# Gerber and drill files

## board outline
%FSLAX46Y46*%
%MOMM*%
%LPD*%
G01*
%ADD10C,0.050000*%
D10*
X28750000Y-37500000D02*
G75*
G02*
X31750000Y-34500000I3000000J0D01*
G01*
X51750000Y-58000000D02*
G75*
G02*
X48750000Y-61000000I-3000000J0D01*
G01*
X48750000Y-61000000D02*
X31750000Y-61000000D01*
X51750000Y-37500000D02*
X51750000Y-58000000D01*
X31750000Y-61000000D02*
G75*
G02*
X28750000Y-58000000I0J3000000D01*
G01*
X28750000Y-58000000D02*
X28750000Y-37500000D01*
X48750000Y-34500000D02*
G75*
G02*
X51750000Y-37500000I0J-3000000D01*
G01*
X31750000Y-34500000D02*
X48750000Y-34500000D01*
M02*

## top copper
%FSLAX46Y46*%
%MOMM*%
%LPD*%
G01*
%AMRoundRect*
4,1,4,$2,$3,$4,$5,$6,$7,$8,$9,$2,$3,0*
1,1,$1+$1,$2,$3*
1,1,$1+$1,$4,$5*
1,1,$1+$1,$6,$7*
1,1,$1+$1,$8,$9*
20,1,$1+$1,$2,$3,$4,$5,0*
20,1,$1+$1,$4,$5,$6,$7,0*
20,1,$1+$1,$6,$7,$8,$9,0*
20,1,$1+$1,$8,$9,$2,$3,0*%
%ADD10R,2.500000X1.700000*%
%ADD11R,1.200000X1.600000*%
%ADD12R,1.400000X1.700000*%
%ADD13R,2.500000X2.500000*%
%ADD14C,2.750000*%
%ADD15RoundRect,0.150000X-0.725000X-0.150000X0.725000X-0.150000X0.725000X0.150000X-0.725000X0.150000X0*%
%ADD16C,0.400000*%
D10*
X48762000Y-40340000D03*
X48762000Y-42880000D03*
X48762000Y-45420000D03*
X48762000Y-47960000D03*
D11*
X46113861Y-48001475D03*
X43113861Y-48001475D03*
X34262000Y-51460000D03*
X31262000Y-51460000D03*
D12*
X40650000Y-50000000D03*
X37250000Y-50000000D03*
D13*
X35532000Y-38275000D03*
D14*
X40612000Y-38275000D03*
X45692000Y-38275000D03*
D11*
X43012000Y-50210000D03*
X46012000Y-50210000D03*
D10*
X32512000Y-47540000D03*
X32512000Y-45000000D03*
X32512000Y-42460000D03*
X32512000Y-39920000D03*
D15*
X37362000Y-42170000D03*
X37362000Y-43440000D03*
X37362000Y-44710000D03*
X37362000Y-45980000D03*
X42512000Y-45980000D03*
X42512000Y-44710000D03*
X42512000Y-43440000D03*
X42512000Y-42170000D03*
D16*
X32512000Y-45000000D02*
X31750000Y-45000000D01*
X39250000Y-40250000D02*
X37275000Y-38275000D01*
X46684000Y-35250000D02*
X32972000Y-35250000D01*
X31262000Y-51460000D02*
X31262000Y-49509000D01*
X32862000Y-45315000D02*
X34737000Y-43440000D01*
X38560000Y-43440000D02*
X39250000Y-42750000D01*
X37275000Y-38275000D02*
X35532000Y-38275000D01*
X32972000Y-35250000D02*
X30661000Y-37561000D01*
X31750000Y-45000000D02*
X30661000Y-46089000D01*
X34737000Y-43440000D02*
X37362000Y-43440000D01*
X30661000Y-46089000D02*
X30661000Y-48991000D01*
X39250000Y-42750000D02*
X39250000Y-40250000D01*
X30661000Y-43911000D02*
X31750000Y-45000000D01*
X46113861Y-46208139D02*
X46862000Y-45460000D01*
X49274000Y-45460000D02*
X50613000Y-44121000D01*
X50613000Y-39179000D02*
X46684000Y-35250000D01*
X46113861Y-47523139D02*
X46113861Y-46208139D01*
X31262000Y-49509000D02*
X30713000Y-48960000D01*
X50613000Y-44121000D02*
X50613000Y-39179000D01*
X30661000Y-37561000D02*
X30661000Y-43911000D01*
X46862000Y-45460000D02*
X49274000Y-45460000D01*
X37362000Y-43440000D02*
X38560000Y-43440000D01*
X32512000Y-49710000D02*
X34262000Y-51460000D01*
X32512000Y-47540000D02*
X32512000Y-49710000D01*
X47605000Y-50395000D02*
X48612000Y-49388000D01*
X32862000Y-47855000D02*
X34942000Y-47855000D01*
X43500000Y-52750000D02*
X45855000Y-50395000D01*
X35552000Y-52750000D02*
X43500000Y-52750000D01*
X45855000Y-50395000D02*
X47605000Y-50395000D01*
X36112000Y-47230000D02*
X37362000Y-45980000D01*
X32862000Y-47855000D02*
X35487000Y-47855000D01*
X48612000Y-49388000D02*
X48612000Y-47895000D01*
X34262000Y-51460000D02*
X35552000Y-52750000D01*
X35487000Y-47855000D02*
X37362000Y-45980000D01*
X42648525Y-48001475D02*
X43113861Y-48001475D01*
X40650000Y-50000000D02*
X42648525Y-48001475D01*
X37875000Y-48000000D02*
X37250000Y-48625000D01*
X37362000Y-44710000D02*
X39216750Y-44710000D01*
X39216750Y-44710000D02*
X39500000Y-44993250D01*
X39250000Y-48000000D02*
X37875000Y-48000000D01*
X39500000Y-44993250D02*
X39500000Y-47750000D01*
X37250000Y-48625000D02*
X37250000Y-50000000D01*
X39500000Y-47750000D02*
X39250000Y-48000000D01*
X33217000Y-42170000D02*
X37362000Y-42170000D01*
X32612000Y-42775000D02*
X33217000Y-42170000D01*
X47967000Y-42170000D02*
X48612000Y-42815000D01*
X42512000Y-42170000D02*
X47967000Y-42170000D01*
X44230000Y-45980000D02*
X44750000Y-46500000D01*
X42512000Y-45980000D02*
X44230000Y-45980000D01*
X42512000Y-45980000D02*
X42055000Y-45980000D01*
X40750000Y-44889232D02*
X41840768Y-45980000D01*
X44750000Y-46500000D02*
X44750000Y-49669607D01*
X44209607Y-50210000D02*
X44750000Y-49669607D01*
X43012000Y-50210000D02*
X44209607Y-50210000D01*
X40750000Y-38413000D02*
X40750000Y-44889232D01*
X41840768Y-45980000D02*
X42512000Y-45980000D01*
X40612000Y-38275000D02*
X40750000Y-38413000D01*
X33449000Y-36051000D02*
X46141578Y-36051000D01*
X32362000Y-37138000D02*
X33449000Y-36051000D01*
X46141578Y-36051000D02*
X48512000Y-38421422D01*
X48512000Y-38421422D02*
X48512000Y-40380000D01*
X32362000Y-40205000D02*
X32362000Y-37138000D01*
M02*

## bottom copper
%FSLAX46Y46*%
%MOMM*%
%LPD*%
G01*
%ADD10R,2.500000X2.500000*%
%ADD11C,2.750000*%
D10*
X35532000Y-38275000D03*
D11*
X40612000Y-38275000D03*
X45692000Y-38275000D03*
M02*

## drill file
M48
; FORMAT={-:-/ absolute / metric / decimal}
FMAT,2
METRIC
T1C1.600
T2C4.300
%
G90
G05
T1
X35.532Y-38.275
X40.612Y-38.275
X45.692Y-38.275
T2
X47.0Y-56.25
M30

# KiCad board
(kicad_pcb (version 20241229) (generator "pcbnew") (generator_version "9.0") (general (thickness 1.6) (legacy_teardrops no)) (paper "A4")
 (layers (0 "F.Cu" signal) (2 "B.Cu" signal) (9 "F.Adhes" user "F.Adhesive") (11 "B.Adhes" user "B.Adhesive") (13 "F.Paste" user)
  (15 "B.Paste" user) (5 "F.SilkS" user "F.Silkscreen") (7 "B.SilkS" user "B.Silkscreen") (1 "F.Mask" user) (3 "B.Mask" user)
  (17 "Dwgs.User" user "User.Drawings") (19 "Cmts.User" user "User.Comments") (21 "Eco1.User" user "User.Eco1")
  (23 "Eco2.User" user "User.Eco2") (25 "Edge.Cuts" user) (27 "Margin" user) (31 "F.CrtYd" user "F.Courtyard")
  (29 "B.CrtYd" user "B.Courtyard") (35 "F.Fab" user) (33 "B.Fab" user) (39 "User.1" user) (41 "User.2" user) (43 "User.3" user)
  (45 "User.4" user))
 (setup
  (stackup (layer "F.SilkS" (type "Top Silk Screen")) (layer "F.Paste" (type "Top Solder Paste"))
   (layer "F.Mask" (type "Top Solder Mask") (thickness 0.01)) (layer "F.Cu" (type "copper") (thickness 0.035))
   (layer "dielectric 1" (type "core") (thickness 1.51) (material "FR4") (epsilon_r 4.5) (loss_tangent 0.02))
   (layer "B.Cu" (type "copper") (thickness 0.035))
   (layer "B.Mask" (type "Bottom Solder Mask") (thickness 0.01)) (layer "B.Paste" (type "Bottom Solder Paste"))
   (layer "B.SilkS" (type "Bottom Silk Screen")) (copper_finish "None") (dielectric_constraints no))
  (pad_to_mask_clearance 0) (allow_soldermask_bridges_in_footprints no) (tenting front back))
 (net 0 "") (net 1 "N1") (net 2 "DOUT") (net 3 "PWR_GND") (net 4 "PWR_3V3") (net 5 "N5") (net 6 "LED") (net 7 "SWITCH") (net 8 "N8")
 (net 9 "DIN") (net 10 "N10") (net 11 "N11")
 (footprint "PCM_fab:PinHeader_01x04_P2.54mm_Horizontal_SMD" (layer "F.Cu") (at 48.762 40.34)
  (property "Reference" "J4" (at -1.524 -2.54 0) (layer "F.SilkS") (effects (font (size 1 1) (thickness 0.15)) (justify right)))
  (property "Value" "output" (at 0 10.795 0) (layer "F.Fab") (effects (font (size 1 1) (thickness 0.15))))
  (pad "1" smd rect (at 0 0) (size 2.5 1.7) (layers "F.Cu" "F.Mask" "F.Paste") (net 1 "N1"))
  (pad "2" smd rect (at 0 2.54) (size 2.5 1.7) (layers "F.Cu" "F.Mask" "F.Paste") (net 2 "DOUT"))
  (pad "3" smd rect (at 0 5.08) (size 2.5 1.7) (layers "F.Cu" "F.Mask" "F.Paste") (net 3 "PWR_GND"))
  (pad "4" smd rect (at 0 7.62) (size 2.5 1.7) (layers "F.Cu" "F.Mask" "F.Paste") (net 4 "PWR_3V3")))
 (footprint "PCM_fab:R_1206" (layer "F.Cu") (at 44.613861 48.001475 180)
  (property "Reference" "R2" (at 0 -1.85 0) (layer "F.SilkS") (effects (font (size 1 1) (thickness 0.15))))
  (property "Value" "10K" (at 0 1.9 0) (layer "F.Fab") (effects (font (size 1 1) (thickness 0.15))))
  (pad "1" smd rect (at -1.5 0 180) (size 1.2 1.6) (layers "F.Cu" "F.Mask" "F.Paste") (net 3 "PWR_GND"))
  (pad "2" smd rect (at 1.5 0 180) (size 1.2 1.6) (layers "F.Cu" "F.Mask" "F.Paste") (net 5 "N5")))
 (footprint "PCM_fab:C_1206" (layer "F.Cu") (at 32.762 51.46 180)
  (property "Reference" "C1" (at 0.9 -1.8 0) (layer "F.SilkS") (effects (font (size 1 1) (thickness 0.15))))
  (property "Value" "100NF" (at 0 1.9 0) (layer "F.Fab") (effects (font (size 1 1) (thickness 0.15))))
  (pad "1" smd rect (at -1.5 0 180) (size 1.2 1.6) (layers "F.Cu" "F.Mask" "F.Paste") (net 4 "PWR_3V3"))
  (pad "2" smd rect (at 1.5 0 180) (size 1.2 1.6) (layers "F.Cu" "F.Mask" "F.Paste") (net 3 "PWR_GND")))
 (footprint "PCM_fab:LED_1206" (layer "F.Cu") (at 38.95 50 180)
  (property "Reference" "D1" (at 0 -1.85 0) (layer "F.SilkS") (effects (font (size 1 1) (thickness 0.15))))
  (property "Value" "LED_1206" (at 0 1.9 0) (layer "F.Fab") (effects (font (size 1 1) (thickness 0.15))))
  (pad "1" smd rect (at -1.7 0 180) (size 1.4 1.7) (layers "F.Cu" "F.Mask" "F.Paste") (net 5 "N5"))
  (pad "2" smd rect (at 1.7 0 180) (size 1.4 1.7) (layers "F.Cu" "F.Mask" "F.Paste") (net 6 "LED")))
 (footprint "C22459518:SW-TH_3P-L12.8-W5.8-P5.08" (layer "F.Cu") (at 40.612 38.275)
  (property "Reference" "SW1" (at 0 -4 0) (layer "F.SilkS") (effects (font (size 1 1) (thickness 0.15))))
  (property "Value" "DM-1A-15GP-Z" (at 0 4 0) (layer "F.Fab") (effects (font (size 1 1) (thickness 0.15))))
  (pad "1" thru_hole rect (at -5.08 0) (size 2.5 2.5) (drill 1.6) (layers "*.Cu" "*.Mask") (remove_unused_layers no) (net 3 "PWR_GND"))
  (pad "2" thru_hole circle (at 0 0) (size 2.75 2.75) (drill 1.6) (layers "*.Cu" "*.Mask") (remove_unused_layers no) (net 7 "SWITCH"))
  (pad "3" thru_hole circle (at 5.08 0) (size 2.75 2.75) (drill 1.6) (layers "*.Cu" "*.Mask") (remove_unused_layers no) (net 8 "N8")))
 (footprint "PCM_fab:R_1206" (layer "F.Cu") (at 44.512 50.21)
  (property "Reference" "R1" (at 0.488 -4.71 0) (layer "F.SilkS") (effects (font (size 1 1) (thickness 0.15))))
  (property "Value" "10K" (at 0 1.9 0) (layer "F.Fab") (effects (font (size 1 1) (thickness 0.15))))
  (pad "1" smd rect (at -1.5 0) (size 1.2 1.6) (layers "F.Cu" "F.Mask" "F.Paste") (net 7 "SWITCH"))
  (pad "2" smd rect (at 1.5 0) (size 1.2 1.6) (layers "F.Cu" "F.Mask" "F.Paste") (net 4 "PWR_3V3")))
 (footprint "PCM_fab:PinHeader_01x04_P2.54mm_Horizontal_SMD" (layer "F.Cu") (at 32.512 47.54 180)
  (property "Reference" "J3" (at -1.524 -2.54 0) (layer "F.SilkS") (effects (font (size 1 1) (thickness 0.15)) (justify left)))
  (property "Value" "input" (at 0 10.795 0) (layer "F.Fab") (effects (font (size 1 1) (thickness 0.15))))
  (pad "1" smd rect (at 0 0 180) (size 2.5 1.7) (layers "F.Cu" "F.Mask" "F.Paste") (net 4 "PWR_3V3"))
  (pad "2" smd rect (at 0 2.54 180) (size 2.5 1.7) (layers "F.Cu" "F.Mask" "F.Paste") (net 3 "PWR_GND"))
  (pad "3" smd rect (at 0 5.08 180) (size 2.5 1.7) (layers "F.Cu" "F.Mask" "F.Paste") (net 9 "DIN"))
  (pad "4" smd rect (at 0 7.62 180) (size 2.5 1.7) (layers "F.Cu" "F.Mask" "F.Paste") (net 1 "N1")))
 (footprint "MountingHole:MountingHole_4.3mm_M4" (layer "F.Cu") (at 47 56.25)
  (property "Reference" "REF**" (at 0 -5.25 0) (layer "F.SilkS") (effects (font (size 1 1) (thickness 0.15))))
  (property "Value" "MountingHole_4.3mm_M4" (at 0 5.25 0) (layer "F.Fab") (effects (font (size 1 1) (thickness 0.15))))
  (pad "" np_thru_hole circle (at 0 0) (size 4.3 4.3) (drill 4.3) (layers "*.Cu" "*.Mask")))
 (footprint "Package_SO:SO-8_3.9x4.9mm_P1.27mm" (layer "F.Cu") (at 39.937 44.075)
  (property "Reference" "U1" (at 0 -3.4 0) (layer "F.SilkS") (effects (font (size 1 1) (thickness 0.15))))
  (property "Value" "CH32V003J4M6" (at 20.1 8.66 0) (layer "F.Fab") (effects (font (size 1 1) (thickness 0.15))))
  (pad "1" smd roundrect (at -2.575 -1.905) (size 1.75 0.6) (layers "F.Cu" "F.Mask" "F.Paste") (roundrect_rratio 0.25) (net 9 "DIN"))
  (pad "2" smd roundrect (at -2.575 -0.635) (size 1.75 0.6) (layers "F.Cu" "F.Mask" "F.Paste") (roundrect_rratio 0.25) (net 3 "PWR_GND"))
  (pad "3" smd roundrect (at -2.575 0.635) (size 1.75 0.6) (layers "F.Cu" "F.Mask" "F.Paste") (roundrect_rratio 0.25) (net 6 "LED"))
  (pad "4" smd roundrect (at -2.575 1.905) (size 1.75 0.6) (layers "F.Cu" "F.Mask" "F.Paste") (roundrect_rratio 0.25) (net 4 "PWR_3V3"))
  (pad "5" smd roundrect (at 2.575 1.905) (size 1.75 0.6) (layers "F.Cu" "F.Mask" "F.Paste") (roundrect_rratio 0.25) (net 7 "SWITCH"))
  (pad "6" smd roundrect (at 2.575 0.635) (size 1.75 0.6) (layers "F.Cu" "F.Mask" "F.Paste") (roundrect_rratio 0.25) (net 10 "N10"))
  (pad "7" smd roundrect (at 2.575 -0.635) (size 1.75 0.6) (layers "F.Cu" "F.Mask" "F.Paste") (roundrect_rratio 0.25) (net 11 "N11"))
  (pad "8" smd roundrect (at 2.575 -1.905) (size 1.75 0.6) (layers "F.Cu" "F.Mask" "F.Paste") (roundrect_rratio 0.25) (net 2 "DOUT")))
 (gr_arc (start 28.75 37.5) (mid 29.62868 35.37868) (end 31.75 34.5) (stroke (width 0.05) (type default)) (layer "Edge.Cuts"))
 (gr_arc (start 51.75 58) (mid 50.87132 60.12132) (end 48.75 61) (stroke (width 0.05) (type default)) (layer "Edge.Cuts"))
 (gr_line (start 48.75 61) (end 31.75 61) (stroke (width 0.05) (type default)) (layer "Edge.Cuts"))
 (gr_line (start 51.75 37.5) (end 51.75 58) (stroke (width 0.05) (type default)) (layer "Edge.Cuts"))
 (gr_arc (start 31.75 61) (mid 29.62868 60.12132) (end 28.75 58) (stroke (width 0.05) (type default)) (layer "Edge.Cuts"))
 (gr_line (start 28.75 58) (end 28.75 37.5) (stroke (width 0.05) (type default)) (layer "Edge.Cuts"))
 (gr_arc (start 48.75 34.5) (mid 50.87132 35.37868) (end 51.75 37.5) (stroke (width 0.05) (type default)) (layer "Edge.Cuts"))
 (gr_line (start 31.75 34.5) (end 48.75 34.5) (stroke (width 0.05) (type default)) (layer "Edge.Cuts"))
 (segment (start 32.512 45) (end 31.75 45) (width 0.4) (layer "F.Cu") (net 3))
 (segment (start 39.25 40.25) (end 37.275 38.275) (width 0.4) (layer "F.Cu") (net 3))
 (segment (start 46.684 35.25) (end 32.972 35.25) (width 0.4) (layer "F.Cu") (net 3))
 (segment (start 31.262 51.46) (end 31.262 49.509) (width 0.4) (layer "F.Cu") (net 3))
 (segment (start 32.862 45.315) (end 34.737 43.44) (width 0.4) (layer "F.Cu") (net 3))
 (segment (start 38.56 43.44) (end 39.25 42.75) (width 0.4) (layer "F.Cu") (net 3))
 (segment (start 37.275 38.275) (end 35.532 38.275) (width 0.4) (layer "F.Cu") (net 3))
 (segment (start 32.972 35.25) (end 30.661 37.561) (width 0.4) (layer "F.Cu") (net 3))
 (segment (start 31.75 45) (end 30.661 46.089) (width 0.4) (layer "F.Cu") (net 3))
 (segment (start 34.737 43.44) (end 37.362 43.44) (width 0.4) (layer "F.Cu") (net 3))
 (segment (start 30.661 46.089) (end 30.661 48.991) (width 0.4) (layer "F.Cu") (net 3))
 (segment (start 39.25 42.75) (end 39.25 40.25) (width 0.4) (layer "F.Cu") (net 3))
 (segment (start 30.661 43.911) (end 31.75 45) (width 0.4) (layer "F.Cu") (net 3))
 (segment (start 46.113861 46.208139) (end 46.862 45.46) (width 0.4) (layer "F.Cu") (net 3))
 (segment (start 49.274 45.46) (end 50.613 44.121) (width 0.4) (layer "F.Cu") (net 3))
 (segment (start 50.613 39.179) (end 46.684 35.25) (width 0.4) (layer "F.Cu") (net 3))
 (segment (start 46.113861 47.523139) (end 46.113861 46.208139) (width 0.4) (layer "F.Cu") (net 3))
 (segment (start 31.262 49.509) (end 30.713 48.96) (width 0.4) (layer "F.Cu") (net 3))
 (segment (start 50.613 44.121) (end 50.613 39.179) (width 0.4) (layer "F.Cu") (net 3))
 (segment (start 30.661 37.561) (end 30.661 43.911) (width 0.4) (layer "F.Cu") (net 3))
 (segment (start 46.862 45.46) (end 49.274 45.46) (width 0.4) (layer "F.Cu") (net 3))
 (segment (start 37.362 43.44) (end 38.56 43.44) (width 0.4) (layer "F.Cu") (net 3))
 (segment (start 32.512 49.71) (end 34.262 51.46) (width 0.4) (layer "F.Cu") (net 4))
 (segment (start 32.512 47.54) (end 32.512 49.71) (width 0.4) (layer "F.Cu") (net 4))
 (segment (start 47.605 50.395) (end 48.612 49.388) (width 0.4) (layer "F.Cu") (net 4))
 (segment (start 32.862 47.855) (end 34.942 47.855) (width 0.4) (layer "F.Cu") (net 4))
 (segment (start 43.5 52.75) (end 45.855 50.395) (width 0.4) (layer "F.Cu") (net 4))
 (segment (start 35.552 52.75) (end 43.5 52.75) (width 0.4) (layer "F.Cu") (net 4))
 (segment (start 45.855 50.395) (end 47.605 50.395) (width 0.4) (layer "F.Cu") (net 4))
 (segment (start 36.112 47.23) (end 37.362 45.98) (width 0.4) (layer "F.Cu") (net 4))
 (segment (start 32.862 47.855) (end 35.487 47.855) (width 0.4) (layer "F.Cu") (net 4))
 (segment (start 48.612 49.388) (end 48.612 47.895) (width 0.4) (layer "F.Cu") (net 4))
 (segment (start 34.262 51.46) (end 35.552 52.75) (width 0.4) (layer "F.Cu") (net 4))
 (segment (start 35.487 47.855) (end 37.362 45.98) (width 0.4) (layer "F.Cu") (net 4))
 (segment (start 42.648525 48.001475) (end 43.113861 48.001475) (width 0.4) (layer "F.Cu") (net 5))
 (segment (start 40.65 50) (end 42.648525 48.001475) (width 0.4) (layer "F.Cu") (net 5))
 (segment (start 37.875 48) (end 37.25 48.625) (width 0.4) (layer "F.Cu") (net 6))
 (segment (start 37.362 44.71) (end 39.21675 44.71) (width 0.4) (layer "F.Cu") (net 6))
 (segment (start 39.21675 44.71) (end 39.5 44.99325) (width 0.4) (layer "F.Cu") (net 6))
 (segment (start 39.25 48) (end 37.875 48) (width 0.4) (layer "F.Cu") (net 6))
 (segment (start 39.5 44.99325) (end 39.5 47.75) (width 0.4) (layer "F.Cu") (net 6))
 (segment (start 37.25 48.625) (end 37.25 50) (width 0.4) (layer "F.Cu") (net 6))
 (segment (start 39.5 47.75) (end 39.25 48) (width 0.4) (layer "F.Cu") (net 6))
 (segment (start 33.217 42.17) (end 37.362 42.17) (width 0.4) (layer "F.Cu") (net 9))
 (segment (start 32.612 42.775) (end 33.217 42.17) (width 0.4) (layer "F.Cu") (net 9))
 (segment (start 47.967 42.17) (end 48.612 42.815) (width 0.4) (layer "F.Cu") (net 2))
 (segment (start 42.512 42.17) (end 47.967 42.17) (width 0.4) (layer "F.Cu") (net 2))
 (segment (start 44.23 45.98) (end 44.75 46.5) (width 0.4) (layer "F.Cu") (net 7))
 (segment (start 42.512 45.98) (end 44.23 45.98) (width 0.4) (layer "F.Cu") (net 7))
 (segment (start 42.512 45.98) (end 42.055 45.98) (width 0.4) (layer "F.Cu") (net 7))
 (segment (start 40.75 44.889232) (end 41.840768 45.98) (width 0.4) (layer "F.Cu") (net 7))
 (segment (start 44.75 46.5) (end 44.75 49.669607) (width 0.4) (layer "F.Cu") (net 7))
 (segment (start 44.209607 50.21) (end 44.75 49.669607) (width 0.4) (layer "F.Cu") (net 7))
 (segment (start 43.012 50.21) (end 44.209607 50.21) (width 0.4) (layer "F.Cu") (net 7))
 (segment (start 40.75 38.413) (end 40.75 44.889232) (width 0.4) (layer "F.Cu") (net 7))
 (segment (start 41.840768 45.98) (end 42.512 45.98) (width 0.4) (layer "F.Cu") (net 7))
 (segment (start 40.612 38.275) (end 40.75 38.413) (width 0.4) (layer "F.Cu") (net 7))
 (segment (start 33.449 36.051) (end 46.141578 36.051) (width 0.4) (layer "F.Cu") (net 1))
 (segment (start 32.362 37.138) (end 33.449 36.051) (width 0.4) (layer "F.Cu") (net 1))
 (segment (start 46.141578 36.051) (end 48.512 38.421422) (width 0.4) (layer "F.Cu") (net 1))
 (segment (start 48.512 38.421422) (end 48.512 40.38) (width 0.4) (layer "F.Cu") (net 1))
 (segment (start 32.362 40.205) (end 32.362 37.138) (width 0.4) (layer "F.Cu") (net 1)))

